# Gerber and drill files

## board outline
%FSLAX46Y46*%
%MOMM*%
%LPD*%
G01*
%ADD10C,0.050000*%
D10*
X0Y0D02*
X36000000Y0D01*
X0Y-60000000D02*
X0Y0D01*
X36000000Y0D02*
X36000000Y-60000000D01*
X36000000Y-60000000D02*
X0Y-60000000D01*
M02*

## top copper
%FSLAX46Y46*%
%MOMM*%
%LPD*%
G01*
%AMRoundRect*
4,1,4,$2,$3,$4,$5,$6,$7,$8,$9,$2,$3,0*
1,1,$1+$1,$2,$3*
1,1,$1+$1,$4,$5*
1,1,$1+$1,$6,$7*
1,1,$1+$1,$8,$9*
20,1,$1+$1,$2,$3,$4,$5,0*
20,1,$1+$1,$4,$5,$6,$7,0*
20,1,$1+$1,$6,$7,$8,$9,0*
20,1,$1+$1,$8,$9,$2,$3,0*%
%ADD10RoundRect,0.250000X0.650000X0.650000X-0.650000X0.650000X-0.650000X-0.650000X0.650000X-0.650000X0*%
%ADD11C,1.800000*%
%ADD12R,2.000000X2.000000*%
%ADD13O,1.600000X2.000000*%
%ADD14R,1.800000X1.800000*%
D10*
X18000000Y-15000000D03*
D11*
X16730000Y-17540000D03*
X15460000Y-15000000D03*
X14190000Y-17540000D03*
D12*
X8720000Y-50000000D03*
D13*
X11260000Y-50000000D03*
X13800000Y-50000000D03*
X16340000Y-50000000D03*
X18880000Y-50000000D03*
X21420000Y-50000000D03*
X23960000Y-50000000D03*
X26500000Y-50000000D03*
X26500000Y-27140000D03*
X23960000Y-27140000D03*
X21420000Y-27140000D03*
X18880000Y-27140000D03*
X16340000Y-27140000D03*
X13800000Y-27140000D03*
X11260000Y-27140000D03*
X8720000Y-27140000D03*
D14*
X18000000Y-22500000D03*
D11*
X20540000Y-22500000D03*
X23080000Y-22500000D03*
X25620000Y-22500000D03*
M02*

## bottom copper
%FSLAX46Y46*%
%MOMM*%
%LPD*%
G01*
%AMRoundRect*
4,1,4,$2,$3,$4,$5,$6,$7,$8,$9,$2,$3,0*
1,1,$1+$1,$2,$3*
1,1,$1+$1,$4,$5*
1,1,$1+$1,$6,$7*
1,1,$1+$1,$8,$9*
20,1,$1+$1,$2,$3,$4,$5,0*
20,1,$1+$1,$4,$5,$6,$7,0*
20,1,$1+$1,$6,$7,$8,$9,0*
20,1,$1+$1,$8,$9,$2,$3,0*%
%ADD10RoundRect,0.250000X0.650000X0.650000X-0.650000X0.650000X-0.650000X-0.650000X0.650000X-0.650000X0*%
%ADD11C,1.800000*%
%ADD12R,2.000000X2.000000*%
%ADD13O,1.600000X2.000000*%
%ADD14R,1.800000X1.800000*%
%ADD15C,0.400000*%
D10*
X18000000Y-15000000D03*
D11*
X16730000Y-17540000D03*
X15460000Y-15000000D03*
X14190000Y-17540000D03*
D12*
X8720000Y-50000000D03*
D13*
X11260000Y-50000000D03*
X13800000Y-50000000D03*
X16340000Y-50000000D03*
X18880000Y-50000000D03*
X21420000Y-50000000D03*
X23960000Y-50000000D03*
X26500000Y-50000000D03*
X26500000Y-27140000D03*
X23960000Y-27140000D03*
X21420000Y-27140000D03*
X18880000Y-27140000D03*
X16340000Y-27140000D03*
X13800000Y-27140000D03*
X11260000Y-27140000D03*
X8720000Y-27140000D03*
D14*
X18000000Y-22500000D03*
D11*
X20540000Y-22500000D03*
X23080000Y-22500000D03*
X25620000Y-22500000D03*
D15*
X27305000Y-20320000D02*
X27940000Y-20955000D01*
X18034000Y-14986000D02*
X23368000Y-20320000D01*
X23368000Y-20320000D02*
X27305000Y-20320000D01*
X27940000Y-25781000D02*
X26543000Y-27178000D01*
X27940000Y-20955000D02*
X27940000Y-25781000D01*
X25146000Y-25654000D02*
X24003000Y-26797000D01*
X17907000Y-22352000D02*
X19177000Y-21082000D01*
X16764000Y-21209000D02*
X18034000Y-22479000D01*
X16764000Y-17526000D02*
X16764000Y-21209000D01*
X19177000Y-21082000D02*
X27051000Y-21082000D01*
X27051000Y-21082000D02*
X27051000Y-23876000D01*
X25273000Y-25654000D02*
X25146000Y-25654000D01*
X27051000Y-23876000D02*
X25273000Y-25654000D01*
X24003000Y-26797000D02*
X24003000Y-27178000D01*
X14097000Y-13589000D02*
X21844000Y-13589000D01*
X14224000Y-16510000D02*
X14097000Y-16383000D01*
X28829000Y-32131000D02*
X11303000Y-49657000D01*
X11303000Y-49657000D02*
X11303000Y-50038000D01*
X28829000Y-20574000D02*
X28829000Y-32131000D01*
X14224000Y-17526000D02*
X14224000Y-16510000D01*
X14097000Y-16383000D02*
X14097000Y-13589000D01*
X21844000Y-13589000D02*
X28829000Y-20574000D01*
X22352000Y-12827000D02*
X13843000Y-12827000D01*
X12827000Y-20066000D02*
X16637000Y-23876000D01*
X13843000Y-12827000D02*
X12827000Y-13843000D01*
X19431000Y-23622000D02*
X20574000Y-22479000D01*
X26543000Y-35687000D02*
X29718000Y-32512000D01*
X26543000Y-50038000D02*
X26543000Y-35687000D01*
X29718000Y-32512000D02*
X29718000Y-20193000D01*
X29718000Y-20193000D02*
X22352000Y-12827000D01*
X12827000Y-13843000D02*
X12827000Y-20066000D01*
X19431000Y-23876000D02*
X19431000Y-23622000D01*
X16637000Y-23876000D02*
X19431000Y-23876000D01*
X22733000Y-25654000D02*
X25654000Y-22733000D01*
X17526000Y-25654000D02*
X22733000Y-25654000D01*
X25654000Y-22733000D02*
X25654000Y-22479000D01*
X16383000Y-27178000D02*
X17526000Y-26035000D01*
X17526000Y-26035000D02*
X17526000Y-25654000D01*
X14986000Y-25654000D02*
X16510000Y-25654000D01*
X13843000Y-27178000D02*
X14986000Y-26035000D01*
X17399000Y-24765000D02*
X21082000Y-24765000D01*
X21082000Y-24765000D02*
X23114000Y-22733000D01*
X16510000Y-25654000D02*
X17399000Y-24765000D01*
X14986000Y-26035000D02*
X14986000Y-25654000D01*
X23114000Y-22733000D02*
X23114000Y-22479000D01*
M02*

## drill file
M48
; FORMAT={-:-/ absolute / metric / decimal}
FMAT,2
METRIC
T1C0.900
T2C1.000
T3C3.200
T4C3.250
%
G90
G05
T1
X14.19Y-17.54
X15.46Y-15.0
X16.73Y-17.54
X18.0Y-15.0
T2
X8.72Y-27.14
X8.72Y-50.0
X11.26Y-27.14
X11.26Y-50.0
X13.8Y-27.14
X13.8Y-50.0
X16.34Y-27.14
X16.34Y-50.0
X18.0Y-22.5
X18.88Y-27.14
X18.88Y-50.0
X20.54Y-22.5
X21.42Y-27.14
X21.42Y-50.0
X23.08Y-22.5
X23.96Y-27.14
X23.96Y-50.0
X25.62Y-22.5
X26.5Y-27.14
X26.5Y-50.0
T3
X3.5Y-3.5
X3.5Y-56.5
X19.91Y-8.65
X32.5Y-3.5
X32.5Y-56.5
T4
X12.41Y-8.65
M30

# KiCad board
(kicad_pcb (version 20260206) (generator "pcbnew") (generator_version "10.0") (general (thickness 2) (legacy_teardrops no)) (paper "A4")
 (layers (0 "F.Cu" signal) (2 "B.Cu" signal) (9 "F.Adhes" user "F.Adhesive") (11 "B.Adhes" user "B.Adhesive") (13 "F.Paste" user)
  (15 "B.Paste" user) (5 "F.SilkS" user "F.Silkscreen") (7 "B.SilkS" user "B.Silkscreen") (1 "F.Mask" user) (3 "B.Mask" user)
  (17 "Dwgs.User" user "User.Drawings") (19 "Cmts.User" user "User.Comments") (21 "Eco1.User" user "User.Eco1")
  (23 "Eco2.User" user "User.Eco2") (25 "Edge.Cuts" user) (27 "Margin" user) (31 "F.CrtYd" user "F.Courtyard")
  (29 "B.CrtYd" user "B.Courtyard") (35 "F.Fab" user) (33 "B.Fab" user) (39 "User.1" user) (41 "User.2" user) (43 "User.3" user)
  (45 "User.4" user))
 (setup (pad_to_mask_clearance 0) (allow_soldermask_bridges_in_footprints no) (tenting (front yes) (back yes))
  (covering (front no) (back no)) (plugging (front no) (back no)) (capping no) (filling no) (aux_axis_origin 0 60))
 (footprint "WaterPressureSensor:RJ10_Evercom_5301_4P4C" (layer "F.Cu") (at 18 15 180)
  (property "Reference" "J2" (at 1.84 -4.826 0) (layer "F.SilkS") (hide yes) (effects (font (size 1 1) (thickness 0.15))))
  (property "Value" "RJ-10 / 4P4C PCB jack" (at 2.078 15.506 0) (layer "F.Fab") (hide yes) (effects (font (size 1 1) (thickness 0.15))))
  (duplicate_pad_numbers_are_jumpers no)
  (pad "" np_thru_hole circle (at -1.91 6.35 180) (size 3.25 3.25) (drill 3.2) (layers "*.Mask"))
  (pad "" np_thru_hole circle (at 5.59 6.35 180) (size 3.25 3.25) (drill 3.25) (layers "*.Mask"))
  (pad "1" thru_hole roundrect (at 0 0 180) (size 1.8 1.8) (drill 0.9) (layers "*.Cu") (remove_unused_layers no)
   (roundrect_rratio 0.1388888889) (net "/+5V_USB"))
  (pad "2" thru_hole circle (at 1.27 -2.54 180) (size 1.8 1.8) (drill 0.9) (layers "*.Cu") (remove_unused_layers no) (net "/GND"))
  (pad "3" thru_hole circle (at 2.54 0 180) (size 1.8 1.8) (drill 0.9) (layers "*.Cu") (remove_unused_layers no)
   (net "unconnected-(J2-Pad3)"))
  (pad "4" thru_hole circle (at 3.81 -2.54 180) (size 1.8 1.8) (drill 0.9) (layers "*.Cu") (remove_unused_layers no) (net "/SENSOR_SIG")))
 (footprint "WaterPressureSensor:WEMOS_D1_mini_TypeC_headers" (layer "F.Cu") (at 8.72 50 90)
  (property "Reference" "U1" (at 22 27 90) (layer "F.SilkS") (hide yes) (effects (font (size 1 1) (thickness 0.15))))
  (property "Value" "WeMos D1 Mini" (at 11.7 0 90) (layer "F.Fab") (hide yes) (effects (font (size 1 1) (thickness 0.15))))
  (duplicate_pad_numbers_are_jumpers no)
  (pad "1" thru_hole rect (at 0 0 90) (size 2 2) (drill 1) (layers "*.Cu") (remove_unused_layers no) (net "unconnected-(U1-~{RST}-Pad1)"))
  (pad "2" thru_hole oval (at 0 2.54 90) (size 2 1.6) (drill 1) (layers "*.Cu") (remove_unused_layers no) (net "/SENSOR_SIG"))
  (pad "3" thru_hole oval (at 0 5.08 90) (size 2 1.6) (drill 1) (layers "*.Cu") (remove_unused_layers no) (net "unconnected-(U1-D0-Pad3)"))
  (pad "4" thru_hole oval (at 0 7.62 90) (size 2 1.6) (drill 1) (layers "*.Cu") (remove_unused_layers no)
   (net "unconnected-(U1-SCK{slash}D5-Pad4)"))
  (pad "5" thru_hole oval (at 0 10.16 90) (size 2 1.6) (drill 1) (layers "*.Cu") (remove_unused_layers no)
   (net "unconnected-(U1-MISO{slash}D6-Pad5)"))
  (pad "6" thru_hole oval (at 0 12.7 90) (size 2 1.6) (drill 1) (layers "*.Cu") (remove_unused_layers no)
   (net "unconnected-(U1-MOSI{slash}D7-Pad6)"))
  (pad "7" thru_hole oval (at 0 15.24 90) (size 2 1.6) (drill 1) (layers "*.Cu") (remove_unused_layers no)
   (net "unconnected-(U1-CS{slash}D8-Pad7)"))
  (pad "8" thru_hole oval (at 0 17.78 90) (size 2 1.6) (drill 1) (layers "*.Cu") (remove_unused_layers no) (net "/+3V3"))
  (pad "9" thru_hole oval (at 22.86 17.78 90) (size 2 1.6) (drill 1) (layers "*.Cu") (remove_unused_layers no) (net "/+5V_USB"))
  (pad "10" thru_hole oval (at 22.86 15.24 90) (size 2 1.6) (drill 1) (layers "*.Cu") (remove_unused_layers no) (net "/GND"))
  (pad "11" thru_hole oval (at 22.86 12.7 90) (size 2 1.6) (drill 1) (layers "*.Cu") (remove_unused_layers no)
   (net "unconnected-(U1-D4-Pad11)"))
  (pad "12" thru_hole oval (at 22.86 10.16 90) (size 2 1.6) (drill 1) (layers "*.Cu") (remove_unused_layers no)
   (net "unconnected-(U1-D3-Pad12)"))
  (pad "13" thru_hole oval (at 22.86 7.62 90) (size 2 1.6) (drill 1) (layers "*.Cu") (remove_unused_layers no) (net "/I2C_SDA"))
  (pad "14" thru_hole oval (at 22.86 5.08 90) (size 2 1.6) (drill 1) (layers "*.Cu") (remove_unused_layers no) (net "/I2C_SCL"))
  (pad "15" thru_hole oval (at 22.86 2.54 90) (size 2 1.6) (drill 1) (layers "*.Cu") (remove_unused_layers no)
   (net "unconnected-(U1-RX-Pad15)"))
  (pad "16" thru_hole oval (at 22.86 0 90) (size 2 1.6) (drill 1) (layers "*.Cu") (remove_unused_layers no)
   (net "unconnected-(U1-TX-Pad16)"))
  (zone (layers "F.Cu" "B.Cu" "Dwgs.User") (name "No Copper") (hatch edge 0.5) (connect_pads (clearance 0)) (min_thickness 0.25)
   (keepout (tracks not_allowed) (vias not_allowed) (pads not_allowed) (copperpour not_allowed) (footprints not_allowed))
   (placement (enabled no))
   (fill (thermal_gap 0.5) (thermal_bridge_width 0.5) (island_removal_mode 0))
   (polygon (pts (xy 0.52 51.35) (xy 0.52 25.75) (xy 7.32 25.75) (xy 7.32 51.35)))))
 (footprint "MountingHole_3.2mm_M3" (layer "F.Cu") (at 32.5 3.5)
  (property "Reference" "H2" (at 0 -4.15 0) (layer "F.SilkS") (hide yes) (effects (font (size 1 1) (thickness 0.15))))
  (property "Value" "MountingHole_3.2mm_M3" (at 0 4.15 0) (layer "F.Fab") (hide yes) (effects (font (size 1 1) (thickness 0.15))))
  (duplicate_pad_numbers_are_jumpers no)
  (pad "" np_thru_hole circle (at 0 0) (size 3.2 3.2) (drill 3.2) (layers "*.Cu" "F.Mask")))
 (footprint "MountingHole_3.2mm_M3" (layer "F.Cu") (at 32.5 56.5)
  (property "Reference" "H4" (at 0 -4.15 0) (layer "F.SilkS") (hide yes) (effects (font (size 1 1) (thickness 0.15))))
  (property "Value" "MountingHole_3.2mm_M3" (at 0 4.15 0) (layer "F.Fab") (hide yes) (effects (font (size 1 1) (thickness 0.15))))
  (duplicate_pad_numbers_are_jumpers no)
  (pad "" np_thru_hole circle (at 0 0) (size 3.2 3.2) (drill 3.2) (layers "*.Cu" "F.Mask")))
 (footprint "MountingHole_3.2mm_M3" (layer "F.Cu") (at 3.5 3.5)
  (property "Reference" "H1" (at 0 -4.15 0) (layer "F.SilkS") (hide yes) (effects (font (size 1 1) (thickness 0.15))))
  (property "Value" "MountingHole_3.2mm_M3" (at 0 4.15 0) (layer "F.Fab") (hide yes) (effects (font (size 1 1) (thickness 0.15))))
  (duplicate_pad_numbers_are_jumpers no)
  (pad "" np_thru_hole circle (at 0 0) (size 3.2 3.2) (drill 3.2) (layers "*.Cu" "F.Mask")))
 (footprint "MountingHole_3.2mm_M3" (layer "F.Cu") (at 3.5 56.5)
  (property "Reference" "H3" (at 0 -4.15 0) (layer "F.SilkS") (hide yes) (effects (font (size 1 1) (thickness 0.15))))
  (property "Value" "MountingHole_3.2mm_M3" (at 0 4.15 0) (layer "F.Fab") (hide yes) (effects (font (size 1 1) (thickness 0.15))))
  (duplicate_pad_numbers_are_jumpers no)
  (pad "" np_thru_hole circle (at 0 0) (size 3.2 3.2) (drill 3.2) (layers "*.Cu" "F.Mask")))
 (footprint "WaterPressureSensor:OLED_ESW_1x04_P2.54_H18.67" (layer "F.Cu") (at 18 22.5 90)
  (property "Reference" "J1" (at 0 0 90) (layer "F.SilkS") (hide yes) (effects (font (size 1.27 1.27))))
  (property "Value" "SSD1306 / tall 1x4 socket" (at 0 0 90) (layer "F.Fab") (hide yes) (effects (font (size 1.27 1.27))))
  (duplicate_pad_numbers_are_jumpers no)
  (pad "1" thru_hole rect (at 0 0 90) (size 1.8 1.8) (drill 1) (layers "*.Cu") (remove_unused_layers no) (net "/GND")
   (thermal_bridge_angle 45))
  (pad "2" thru_hole circle (at 0 2.54 90) (size 1.8 1.8) (drill 1) (layers "*.Cu") (remove_unused_layers no) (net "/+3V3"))
  (pad "3" thru_hole circle (at 0 5.08 90) (size 1.8 1.8) (drill 1) (layers "*.Cu") (remove_unused_layers no) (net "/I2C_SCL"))
  (pad "4" thru_hole circle (at 0 7.62 90) (size 1.8 1.8) (drill 1) (layers "*.Cu") (remove_unused_layers no) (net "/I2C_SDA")))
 (gr_line (start 0 0) (end 36 0) (stroke (width 0.05) (type default)) (layer "Edge.Cuts"))
 (gr_line (start 0 60) (end 0 0) (stroke (width 0.05) (type default)) (layer "Edge.Cuts"))
 (gr_line (start 36 0) (end 36 60) (stroke (width 0.05) (type default)) (layer "Edge.Cuts"))
 (gr_line (start 36 60) (end 0 60) (stroke (width 0.05) (type default)) (layer "Edge.Cuts"))
 (segment (start 27.305 20.32) (end 27.94 20.955) (width 0.4) (layer "B.Cu") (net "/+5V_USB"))
 (segment (start 18.034 14.986) (end 23.368 20.32) (width 0.4) (layer "B.Cu") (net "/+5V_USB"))
 (segment (start 23.368 20.32) (end 27.305 20.32) (width 0.4) (layer "B.Cu") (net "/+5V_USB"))
 (segment (start 27.94 25.781) (end 26.543 27.178) (width 0.4) (layer "B.Cu") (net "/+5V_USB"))
 (segment (start 27.94 20.955) (end 27.94 25.781) (width 0.4) (layer "B.Cu") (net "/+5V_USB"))
 (segment (start 25.146 25.654) (end 24.003 26.797) (width 0.4) (layer "B.Cu") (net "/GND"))
 (segment (start 17.907 22.352) (end 19.177 21.082) (width 0.4) (layer "B.Cu") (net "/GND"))
 (segment (start 16.764 21.209) (end 18.034 22.479) (width 0.4) (layer "B.Cu") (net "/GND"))
 (segment (start 16.764 17.526) (end 16.764 21.209) (width 0.4) (layer "B.Cu") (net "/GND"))
 (segment (start 19.177 21.082) (end 27.051 21.082) (width 0.4) (layer "B.Cu") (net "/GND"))
 (segment (start 27.051 21.082) (end 27.051 23.876) (width 0.4) (layer "B.Cu") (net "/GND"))
 (segment (start 25.273 25.654) (end 25.146 25.654) (width 0.4) (layer "B.Cu") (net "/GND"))
 (segment (start 27.051 23.876) (end 25.273 25.654) (width 0.4) (layer "B.Cu") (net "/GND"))
 (segment (start 24.003 26.797) (end 24.003 27.178) (width 0.4) (layer "B.Cu") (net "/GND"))
 (segment (start 14.097 13.589) (end 21.844 13.589) (width 0.4) (layer "B.Cu") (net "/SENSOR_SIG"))
 (segment (start 14.224 16.51) (end 14.097 16.383) (width 0.4) (layer "B.Cu") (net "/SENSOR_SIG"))
 (segment (start 28.829 32.131) (end 11.303 49.657) (width 0.4) (layer "B.Cu") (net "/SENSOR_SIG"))
 (segment (start 11.303 49.657) (end 11.303 50.038) (width 0.4) (layer "B.Cu") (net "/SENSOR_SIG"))
 (segment (start 28.829 20.574) (end 28.829 32.131) (width 0.4) (layer "B.Cu") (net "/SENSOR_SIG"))
 (segment (start 14.224 17.526) (end 14.224 16.51) (width 0.4) (layer "B.Cu") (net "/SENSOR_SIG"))
 (segment (start 14.097 16.383) (end 14.097 13.589) (width 0.4) (layer "B.Cu") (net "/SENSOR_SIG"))
 (segment (start 21.844 13.589) (end 28.829 20.574) (width 0.4) (layer "B.Cu") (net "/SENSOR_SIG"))
 (segment (start 22.352 12.827) (end 13.843 12.827) (width 0.4) (layer "B.Cu") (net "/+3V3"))
 (segment (start 12.827 20.066) (end 16.637 23.876) (width 0.4) (layer "B.Cu") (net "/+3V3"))
 (segment (start 13.843 12.827) (end 12.827 13.843) (width 0.4) (layer "B.Cu") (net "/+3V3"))
 (segment (start 19.431 23.622) (end 20.574 22.479) (width 0.4) (layer "B.Cu") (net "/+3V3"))
 (segment (start 26.543 35.687) (end 29.718 32.512) (width 0.4) (layer "B.Cu") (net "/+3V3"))
 (segment (start 26.543 50.038) (end 26.543 35.687) (width 0.4) (layer "B.Cu") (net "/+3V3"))
 (segment (start 29.718 32.512) (end 29.718 20.193) (width 0.4) (layer "B.Cu") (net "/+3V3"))
 (segment (start 29.718 20.193) (end 22.352 12.827) (width 0.4) (layer "B.Cu") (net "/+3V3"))
 (segment (start 12.827 13.843) (end 12.827 20.066) (width 0.4) (layer "B.Cu") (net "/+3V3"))
 (segment (start 19.431 23.876) (end 19.431 23.622) (width 0.4) (layer "B.Cu") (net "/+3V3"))
 (segment (start 16.637 23.876) (end 19.431 23.876) (width 0.4) (layer "B.Cu") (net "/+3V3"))
 (segment (start 22.733 25.654) (end 25.654 22.733) (width 0.4) (layer "B.Cu") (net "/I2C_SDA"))
 (segment (start 17.526 25.654) (end 22.733 25.654) (width 0.4) (layer "B.Cu") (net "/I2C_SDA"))
 (segment (start 25.654 22.733) (end 25.654 22.479) (width 0.4) (layer "B.Cu") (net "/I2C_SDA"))
 (segment (start 16.383 27.178) (end 17.526 26.035) (width 0.4) (layer "B.Cu") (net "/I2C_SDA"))
 (segment (start 17.526 26.035) (end 17.526 25.654) (width 0.4) (layer "B.Cu") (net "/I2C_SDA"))
 (segment (start 14.986 25.654) (end 16.51 25.654) (width 0.4) (layer "B.Cu") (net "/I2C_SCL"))
 (segment (start 13.843 27.178) (end 14.986 26.035) (width 0.4) (layer "B.Cu") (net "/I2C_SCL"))
 (segment (start 17.399 24.765) (end 21.082 24.765) (width 0.4) (layer "B.Cu") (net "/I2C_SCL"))
 (segment (start 21.082 24.765) (end 23.114 22.733) (width 0.4) (layer "B.Cu") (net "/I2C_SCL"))
 (segment (start 16.51 25.654) (end 17.399 24.765) (width 0.4) (layer "B.Cu") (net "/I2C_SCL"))
 (segment (start 14.986 26.035) (end 14.986 25.654) (width 0.4) (layer "B.Cu") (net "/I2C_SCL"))
 (segment (start 23.114 22.733) (end 23.114 22.479) (width 0.4) (layer "B.Cu") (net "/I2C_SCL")))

